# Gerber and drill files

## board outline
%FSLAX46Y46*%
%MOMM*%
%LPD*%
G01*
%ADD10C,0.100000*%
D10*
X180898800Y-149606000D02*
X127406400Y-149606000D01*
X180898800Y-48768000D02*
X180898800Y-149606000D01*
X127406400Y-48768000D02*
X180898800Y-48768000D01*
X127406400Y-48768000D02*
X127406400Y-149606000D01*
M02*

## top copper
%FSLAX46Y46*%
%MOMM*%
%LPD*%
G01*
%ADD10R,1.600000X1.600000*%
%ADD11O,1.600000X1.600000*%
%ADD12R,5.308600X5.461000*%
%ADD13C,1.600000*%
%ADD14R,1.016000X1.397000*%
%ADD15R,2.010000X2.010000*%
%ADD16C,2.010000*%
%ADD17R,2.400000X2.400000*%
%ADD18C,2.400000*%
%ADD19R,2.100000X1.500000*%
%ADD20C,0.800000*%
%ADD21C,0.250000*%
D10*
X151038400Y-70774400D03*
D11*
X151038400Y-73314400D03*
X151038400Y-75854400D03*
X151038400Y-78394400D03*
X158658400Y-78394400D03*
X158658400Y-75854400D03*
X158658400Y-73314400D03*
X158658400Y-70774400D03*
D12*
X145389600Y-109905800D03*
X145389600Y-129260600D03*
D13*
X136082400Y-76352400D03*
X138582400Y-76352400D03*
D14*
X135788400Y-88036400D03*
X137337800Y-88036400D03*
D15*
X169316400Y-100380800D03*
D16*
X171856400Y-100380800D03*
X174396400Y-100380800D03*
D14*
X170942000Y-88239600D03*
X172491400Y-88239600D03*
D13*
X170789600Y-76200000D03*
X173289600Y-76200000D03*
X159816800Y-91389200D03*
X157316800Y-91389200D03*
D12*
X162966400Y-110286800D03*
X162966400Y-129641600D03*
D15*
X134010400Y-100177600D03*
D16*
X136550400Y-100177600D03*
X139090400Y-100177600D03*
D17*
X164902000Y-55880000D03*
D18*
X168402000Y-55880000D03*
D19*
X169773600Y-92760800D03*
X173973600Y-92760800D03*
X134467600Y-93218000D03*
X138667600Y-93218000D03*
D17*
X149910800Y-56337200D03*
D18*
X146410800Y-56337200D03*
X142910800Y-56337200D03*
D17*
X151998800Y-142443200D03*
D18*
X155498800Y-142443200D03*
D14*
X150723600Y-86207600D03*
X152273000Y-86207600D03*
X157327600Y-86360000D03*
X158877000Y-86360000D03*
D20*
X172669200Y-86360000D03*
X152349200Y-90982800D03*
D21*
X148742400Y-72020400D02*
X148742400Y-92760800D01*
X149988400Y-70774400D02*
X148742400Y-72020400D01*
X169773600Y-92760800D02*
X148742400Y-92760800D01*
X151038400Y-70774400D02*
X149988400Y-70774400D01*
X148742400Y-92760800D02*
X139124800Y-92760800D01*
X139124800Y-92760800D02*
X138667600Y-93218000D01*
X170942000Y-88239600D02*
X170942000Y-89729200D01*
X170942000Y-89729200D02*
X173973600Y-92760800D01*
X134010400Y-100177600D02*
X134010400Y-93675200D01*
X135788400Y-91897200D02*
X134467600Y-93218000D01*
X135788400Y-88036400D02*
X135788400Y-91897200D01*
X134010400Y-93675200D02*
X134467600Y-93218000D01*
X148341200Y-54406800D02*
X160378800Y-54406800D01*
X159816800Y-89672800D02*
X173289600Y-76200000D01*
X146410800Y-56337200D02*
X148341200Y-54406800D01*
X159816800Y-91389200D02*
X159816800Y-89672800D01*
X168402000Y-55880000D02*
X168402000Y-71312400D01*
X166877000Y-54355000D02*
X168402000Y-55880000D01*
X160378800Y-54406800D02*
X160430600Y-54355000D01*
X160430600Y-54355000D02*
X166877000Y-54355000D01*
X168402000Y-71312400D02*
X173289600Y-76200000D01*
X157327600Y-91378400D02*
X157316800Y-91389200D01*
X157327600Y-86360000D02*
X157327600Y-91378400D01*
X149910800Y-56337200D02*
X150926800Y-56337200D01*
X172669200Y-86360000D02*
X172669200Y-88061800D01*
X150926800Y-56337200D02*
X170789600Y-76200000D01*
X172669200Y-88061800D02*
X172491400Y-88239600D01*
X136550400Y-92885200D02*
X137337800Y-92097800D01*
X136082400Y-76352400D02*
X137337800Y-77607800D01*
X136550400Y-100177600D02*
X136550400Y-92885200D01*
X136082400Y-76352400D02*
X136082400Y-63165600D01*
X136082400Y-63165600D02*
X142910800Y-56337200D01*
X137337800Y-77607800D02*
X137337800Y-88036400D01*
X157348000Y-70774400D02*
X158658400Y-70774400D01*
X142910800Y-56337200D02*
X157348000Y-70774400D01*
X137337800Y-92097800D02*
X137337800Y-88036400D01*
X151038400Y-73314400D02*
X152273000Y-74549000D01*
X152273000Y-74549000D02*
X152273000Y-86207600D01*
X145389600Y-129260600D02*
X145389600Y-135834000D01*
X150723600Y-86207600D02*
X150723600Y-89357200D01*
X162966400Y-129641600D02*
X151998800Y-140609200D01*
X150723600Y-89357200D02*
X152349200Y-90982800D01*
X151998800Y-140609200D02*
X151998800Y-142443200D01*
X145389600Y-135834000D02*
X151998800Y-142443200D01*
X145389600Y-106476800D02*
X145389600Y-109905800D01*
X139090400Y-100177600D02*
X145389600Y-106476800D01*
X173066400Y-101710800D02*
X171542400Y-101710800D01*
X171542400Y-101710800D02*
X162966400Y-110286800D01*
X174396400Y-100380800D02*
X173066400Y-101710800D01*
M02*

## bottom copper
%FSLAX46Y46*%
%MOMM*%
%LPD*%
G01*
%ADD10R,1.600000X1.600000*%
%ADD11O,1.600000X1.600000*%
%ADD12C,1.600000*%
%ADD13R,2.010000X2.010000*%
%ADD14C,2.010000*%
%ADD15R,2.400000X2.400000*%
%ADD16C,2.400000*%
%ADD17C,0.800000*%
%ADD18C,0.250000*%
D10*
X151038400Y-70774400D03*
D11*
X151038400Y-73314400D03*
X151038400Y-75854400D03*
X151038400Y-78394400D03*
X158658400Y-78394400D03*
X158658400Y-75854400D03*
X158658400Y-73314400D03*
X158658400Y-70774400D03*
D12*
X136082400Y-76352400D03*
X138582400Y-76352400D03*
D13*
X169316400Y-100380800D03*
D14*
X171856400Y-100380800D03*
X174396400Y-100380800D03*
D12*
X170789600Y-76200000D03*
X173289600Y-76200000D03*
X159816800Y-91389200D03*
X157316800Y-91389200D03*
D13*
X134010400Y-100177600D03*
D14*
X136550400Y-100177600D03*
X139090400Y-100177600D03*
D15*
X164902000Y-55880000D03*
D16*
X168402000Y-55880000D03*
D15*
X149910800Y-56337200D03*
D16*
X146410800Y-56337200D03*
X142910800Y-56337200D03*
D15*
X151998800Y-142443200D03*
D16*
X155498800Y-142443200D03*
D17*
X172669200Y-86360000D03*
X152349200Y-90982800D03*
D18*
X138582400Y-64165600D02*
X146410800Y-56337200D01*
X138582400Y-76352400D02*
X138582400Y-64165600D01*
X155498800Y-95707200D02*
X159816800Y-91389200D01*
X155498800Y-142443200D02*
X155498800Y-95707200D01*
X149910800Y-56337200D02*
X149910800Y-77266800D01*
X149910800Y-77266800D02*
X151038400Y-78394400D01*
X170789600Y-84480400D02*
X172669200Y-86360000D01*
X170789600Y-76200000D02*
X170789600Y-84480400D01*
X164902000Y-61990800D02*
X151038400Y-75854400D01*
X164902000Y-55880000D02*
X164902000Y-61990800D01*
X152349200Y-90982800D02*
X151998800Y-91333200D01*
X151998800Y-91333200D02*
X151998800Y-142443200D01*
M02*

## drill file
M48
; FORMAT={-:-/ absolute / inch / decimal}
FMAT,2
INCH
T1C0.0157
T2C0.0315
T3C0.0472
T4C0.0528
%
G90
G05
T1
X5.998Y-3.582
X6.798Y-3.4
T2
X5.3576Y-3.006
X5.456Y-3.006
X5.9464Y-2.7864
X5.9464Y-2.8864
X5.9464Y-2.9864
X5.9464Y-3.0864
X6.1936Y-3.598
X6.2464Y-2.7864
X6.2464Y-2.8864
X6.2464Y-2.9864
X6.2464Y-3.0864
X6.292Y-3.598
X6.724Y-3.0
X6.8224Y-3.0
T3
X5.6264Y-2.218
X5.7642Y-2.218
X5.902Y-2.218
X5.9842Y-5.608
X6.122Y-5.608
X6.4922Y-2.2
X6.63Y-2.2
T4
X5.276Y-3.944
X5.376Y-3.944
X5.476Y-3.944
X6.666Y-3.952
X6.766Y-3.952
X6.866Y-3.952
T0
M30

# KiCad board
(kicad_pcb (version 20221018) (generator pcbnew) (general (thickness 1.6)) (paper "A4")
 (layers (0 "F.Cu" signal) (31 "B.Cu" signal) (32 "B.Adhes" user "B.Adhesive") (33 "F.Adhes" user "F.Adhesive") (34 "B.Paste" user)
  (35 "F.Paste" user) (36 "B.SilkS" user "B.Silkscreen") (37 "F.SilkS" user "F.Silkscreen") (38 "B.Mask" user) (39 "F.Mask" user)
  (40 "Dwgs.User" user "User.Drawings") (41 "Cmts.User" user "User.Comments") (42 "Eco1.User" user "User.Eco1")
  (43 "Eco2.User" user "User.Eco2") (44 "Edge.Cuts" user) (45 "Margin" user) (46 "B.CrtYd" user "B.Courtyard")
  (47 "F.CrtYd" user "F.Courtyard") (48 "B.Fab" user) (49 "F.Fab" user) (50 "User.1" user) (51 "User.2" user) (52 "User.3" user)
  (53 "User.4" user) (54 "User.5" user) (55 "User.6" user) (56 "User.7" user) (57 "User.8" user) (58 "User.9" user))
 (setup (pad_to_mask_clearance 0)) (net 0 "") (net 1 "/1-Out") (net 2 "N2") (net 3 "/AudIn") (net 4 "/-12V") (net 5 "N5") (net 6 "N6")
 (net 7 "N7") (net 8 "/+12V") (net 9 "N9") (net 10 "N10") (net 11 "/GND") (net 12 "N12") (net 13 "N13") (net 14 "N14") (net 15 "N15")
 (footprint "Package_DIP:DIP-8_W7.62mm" (layer "F.Cu") (at 151.0384 70.7744)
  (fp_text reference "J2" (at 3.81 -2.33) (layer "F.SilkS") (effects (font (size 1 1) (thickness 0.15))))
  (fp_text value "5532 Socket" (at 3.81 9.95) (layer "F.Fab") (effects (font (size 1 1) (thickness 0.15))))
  (pad "1" thru_hole rect (at 0 0) (size 1.6 1.6) (drill 0.8) (layers "*.Cu" "*.Mask") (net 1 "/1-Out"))
  (pad "2" thru_hole oval (at 0 2.54) (size 1.6 1.6) (drill 0.8) (layers "*.Cu" "*.Mask") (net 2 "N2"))
  (pad "3" thru_hole oval (at 0 5.08) (size 1.6 1.6) (drill 0.8) (layers "*.Cu" "*.Mask") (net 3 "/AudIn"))
  (pad "4" thru_hole oval (at 0 7.62) (size 1.6 1.6) (drill 0.8) (layers "*.Cu" "*.Mask") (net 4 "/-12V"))
  (pad "5" thru_hole oval (at 7.62 7.62) (size 1.6 1.6) (drill 0.8) (layers "*.Cu" "*.Mask") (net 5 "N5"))
  (pad "6" thru_hole oval (at 7.62 5.08) (size 1.6 1.6) (drill 0.8) (layers "*.Cu" "*.Mask") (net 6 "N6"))
  (pad "7" thru_hole oval (at 7.62 2.54) (size 1.6 1.6) (drill 0.8) (layers "*.Cu" "*.Mask") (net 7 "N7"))
  (pad "8" thru_hole oval (at 7.62 0) (size 1.6 1.6) (drill 0.8) (layers "*.Cu" "*.Mask") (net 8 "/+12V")))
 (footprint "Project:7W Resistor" (layer "F.Cu") (at 145.3896 119.5832 -90)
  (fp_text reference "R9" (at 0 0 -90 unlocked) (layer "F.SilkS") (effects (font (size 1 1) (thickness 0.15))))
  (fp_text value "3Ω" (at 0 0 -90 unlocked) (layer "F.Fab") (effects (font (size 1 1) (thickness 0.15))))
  (pad "1" smd rect (at -9.6774 0) (size 5.3086 5.461) (layers "F.Cu" "F.Paste" "F.Mask") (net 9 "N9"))
  (pad "2" smd rect (at 9.6774 0) (size 5.3086 5.461) (layers "F.Cu" "F.Paste" "F.Mask") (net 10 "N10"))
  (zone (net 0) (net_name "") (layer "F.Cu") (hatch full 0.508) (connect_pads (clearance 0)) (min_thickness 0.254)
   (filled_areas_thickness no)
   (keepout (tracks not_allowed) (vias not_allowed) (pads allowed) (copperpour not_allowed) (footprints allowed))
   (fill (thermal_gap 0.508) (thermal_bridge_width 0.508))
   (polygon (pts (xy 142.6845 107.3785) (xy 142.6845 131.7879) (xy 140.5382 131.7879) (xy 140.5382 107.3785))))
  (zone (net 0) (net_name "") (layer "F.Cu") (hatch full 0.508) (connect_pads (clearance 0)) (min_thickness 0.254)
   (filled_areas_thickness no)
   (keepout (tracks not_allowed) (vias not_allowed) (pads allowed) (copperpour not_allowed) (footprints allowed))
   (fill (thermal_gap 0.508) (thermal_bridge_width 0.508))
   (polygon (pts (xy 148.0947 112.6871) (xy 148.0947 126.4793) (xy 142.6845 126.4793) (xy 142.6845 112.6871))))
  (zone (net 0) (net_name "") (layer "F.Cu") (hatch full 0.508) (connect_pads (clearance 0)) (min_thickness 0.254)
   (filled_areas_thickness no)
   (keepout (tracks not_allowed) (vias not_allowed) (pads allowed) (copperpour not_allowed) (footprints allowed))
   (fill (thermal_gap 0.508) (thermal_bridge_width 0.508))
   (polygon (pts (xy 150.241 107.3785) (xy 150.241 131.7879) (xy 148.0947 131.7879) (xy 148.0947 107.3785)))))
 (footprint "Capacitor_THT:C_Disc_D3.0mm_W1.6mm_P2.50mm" (layer "F.Cu") (at 136.0824 76.3524)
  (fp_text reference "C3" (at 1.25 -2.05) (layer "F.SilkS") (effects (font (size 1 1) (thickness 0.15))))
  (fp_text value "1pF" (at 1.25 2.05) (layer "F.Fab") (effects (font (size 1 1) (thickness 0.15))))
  (pad "1" thru_hole circle (at 0 0) (size 1.6 1.6) (drill 0.8) (layers "*.Cu" "*.Mask") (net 8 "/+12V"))
  (pad "2" thru_hole circle (at 2.5 0) (size 1.6 1.6) (drill 0.8) (layers "*.Cu" "*.Mask") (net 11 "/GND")))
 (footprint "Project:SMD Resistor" (layer "F.Cu") (at 136.5631 88.0364)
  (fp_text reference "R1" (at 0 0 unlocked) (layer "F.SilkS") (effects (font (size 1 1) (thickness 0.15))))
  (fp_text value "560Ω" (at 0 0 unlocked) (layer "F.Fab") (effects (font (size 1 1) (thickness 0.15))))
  (pad "1" smd rect (at -0.7747 0) (size 1.016 1.397) (layers "F.Cu" "F.Paste" "F.Mask") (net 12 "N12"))
  (pad "2" smd rect (at 0.7747 0) (size 1.016 1.397) (layers "F.Cu" "F.Paste" "F.Mask") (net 8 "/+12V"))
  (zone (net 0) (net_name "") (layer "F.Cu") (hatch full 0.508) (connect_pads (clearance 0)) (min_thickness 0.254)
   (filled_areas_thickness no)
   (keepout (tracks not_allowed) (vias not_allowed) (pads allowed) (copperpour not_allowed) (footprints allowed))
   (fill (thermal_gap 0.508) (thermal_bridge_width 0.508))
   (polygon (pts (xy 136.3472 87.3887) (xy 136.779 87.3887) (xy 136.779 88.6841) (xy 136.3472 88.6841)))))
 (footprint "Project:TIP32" (layer "F.Cu") (at 169.3164 100.3808)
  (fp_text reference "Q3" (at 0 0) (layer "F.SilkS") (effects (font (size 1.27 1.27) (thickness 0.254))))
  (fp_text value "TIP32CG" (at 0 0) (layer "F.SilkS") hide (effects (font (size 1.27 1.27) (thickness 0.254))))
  (pad "1" thru_hole rect (at 0 0) (size 2.01 2.01) (drill 1.34) (layers "*.Cu" "*.Mask") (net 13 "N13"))
  (pad "2" thru_hole circle (at 2.54 0) (size 2.01 2.01) (drill 1.34) (layers "*.Cu" "*.Mask") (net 4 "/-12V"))
  (pad "3" thru_hole circle (at 5.08 0) (size 2.01 2.01) (drill 1.34) (layers "*.Cu" "*.Mask") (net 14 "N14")))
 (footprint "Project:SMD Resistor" (layer "F.Cu") (at 171.7167 88.2396)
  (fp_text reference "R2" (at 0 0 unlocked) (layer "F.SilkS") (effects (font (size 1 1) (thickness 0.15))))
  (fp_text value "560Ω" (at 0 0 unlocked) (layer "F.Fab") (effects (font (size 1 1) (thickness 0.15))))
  (pad "1" smd rect (at -0.7747 0) (size 1.016 1.397) (layers "F.Cu" "F.Paste" "F.Mask") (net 13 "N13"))
  (pad "2" smd rect (at 0.7747 0) (size 1.016 1.397) (layers "F.Cu" "F.Paste" "F.Mask") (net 4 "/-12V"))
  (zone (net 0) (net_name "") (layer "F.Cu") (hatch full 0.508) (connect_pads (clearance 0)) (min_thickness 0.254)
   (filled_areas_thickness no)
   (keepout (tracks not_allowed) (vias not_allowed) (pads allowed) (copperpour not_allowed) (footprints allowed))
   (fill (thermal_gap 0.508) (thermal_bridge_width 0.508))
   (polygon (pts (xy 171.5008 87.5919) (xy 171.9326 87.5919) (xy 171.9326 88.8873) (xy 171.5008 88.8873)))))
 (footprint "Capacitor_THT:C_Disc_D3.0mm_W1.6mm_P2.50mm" (layer "F.Cu") (at 170.7896 76.2)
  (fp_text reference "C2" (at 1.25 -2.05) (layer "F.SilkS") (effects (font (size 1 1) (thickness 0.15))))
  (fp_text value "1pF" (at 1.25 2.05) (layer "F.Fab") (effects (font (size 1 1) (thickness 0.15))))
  (pad "1" thru_hole circle (at 0 0) (size 1.6 1.6) (drill 0.8) (layers "*.Cu" "*.Mask") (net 4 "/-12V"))
  (pad "2" thru_hole circle (at 2.5 0) (size 1.6 1.6) (drill 0.8) (layers "*.Cu" "*.Mask") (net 11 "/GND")))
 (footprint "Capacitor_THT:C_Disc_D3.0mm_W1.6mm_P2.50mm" (layer "F.Cu") (at 159.8168 91.3892 180)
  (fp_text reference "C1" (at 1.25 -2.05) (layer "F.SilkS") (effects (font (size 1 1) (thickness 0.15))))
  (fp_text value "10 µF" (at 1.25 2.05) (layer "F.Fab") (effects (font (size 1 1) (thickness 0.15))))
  (pad "1" thru_hole circle (at 0 0 180) (size 1.6 1.6) (drill 0.8) (layers "*.Cu" "*.Mask") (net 11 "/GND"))
  (pad "2" thru_hole circle (at 2.5 0 180) (size 1.6 1.6) (drill 0.8) (layers "*.Cu" "*.Mask") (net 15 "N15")))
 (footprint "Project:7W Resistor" (layer "F.Cu") (at 162.9664 119.9642 -90)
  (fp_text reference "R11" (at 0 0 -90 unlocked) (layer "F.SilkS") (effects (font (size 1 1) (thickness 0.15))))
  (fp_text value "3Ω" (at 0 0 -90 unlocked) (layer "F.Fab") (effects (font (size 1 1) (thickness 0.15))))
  (pad "1" smd rect (at -9.6774 0) (size 5.3086 5.461) (layers "F.Cu" "F.Paste" "F.Mask") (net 14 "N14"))
  (pad "2" smd rect (at 9.6774 0) (size 5.3086 5.461) (layers "F.Cu" "F.Paste" "F.Mask") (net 10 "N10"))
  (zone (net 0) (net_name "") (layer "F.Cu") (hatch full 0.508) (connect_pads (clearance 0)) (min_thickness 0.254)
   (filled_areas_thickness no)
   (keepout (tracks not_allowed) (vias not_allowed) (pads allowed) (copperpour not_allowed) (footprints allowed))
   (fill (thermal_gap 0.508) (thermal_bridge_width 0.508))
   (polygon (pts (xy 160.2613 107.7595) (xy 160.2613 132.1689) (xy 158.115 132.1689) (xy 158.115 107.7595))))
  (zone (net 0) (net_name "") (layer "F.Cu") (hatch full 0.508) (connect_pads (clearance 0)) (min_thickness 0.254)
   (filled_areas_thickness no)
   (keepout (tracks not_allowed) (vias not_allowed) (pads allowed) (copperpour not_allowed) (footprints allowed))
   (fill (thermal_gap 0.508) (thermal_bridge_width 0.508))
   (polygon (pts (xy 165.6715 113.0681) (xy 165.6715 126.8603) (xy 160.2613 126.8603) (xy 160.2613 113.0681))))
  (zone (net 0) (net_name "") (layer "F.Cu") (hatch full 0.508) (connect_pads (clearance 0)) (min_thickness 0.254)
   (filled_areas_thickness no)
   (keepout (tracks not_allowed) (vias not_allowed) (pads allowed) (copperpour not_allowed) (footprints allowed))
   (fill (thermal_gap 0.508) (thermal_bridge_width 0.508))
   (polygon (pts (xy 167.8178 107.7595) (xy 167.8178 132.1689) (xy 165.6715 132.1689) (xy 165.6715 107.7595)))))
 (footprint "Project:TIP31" (layer "F.Cu") (at 134.0104 100.1776)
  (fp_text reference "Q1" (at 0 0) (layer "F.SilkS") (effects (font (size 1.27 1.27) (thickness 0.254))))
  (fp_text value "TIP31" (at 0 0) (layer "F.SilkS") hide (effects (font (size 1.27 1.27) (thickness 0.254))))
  (pad "1" thru_hole rect (at 0 0) (size 2.01 2.01) (drill 1.34) (layers "*.Cu" "*.Mask") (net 12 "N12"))
  (pad "2" thru_hole circle (at 2.54 0) (size 2.01 2.01) (drill 1.34) (layers "*.Cu" "*.Mask") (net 8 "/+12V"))
  (pad "3" thru_hole circle (at 5.08 0) (size 2.01 2.01) (drill 1.34) (layers "*.Cu" "*.Mask") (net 9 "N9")))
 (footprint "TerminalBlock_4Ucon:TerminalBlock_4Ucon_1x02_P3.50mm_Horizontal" (layer "F.Cu") (at 164.902 55.88)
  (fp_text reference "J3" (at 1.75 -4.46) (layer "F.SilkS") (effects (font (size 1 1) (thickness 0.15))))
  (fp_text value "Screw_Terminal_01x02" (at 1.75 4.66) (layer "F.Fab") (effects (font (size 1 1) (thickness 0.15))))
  (pad "1" thru_hole rect (at 0 0) (size 2.4 2.4) (drill 1.2) (layers "*.Cu" "*.Mask") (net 3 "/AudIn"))
  (pad "2" thru_hole circle (at 3.5 0) (size 2.4 2.4) (drill 1.2) (layers "*.Cu" "*.Mask") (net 11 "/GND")))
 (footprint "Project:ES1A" (layer "F.Cu") (at 171.8736 92.7608)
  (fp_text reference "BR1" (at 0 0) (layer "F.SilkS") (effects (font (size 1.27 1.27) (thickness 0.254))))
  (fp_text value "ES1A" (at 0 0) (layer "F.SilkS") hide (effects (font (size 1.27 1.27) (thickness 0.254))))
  (pad "1" smd rect (at -2.1 0 90) (size 1.5 2.1) (layers "F.Cu" "F.Paste" "F.Mask") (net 1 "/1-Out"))
  (pad "2" smd rect (at 2.1 0 90) (size 1.5 2.1) (layers "F.Cu" "F.Paste" "F.Mask") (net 13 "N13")))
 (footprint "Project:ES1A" (layer "F.Cu") (at 136.5676 93.218)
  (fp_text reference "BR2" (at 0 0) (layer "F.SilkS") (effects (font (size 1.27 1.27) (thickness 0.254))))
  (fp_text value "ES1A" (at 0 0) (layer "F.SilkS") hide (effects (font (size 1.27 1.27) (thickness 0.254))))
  (pad "1" smd rect (at -2.1 0 90) (size 1.5 2.1) (layers "F.Cu" "F.Paste" "F.Mask") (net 12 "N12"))
  (pad "2" smd rect (at 2.1 0 90) (size 1.5 2.1) (layers "F.Cu" "F.Paste" "F.Mask") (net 1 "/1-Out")))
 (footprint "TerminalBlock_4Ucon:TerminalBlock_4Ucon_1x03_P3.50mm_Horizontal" (layer "F.Cu") (at 149.9108 56.3372 180)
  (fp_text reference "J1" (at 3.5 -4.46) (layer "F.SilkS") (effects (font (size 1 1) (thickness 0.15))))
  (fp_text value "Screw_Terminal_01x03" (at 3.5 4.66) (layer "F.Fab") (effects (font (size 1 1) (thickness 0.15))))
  (pad "1" thru_hole rect (at 0 0 180) (size 2.4 2.4) (drill 1.2) (layers "*.Cu" "*.Mask") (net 4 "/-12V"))
  (pad "2" thru_hole circle (at 3.5 0 180) (size 2.4 2.4) (drill 1.2) (layers "*.Cu" "*.Mask") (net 11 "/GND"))
  (pad "3" thru_hole circle (at 7 0 180) (size 2.4 2.4) (drill 1.2) (layers "*.Cu" "*.Mask") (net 8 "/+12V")))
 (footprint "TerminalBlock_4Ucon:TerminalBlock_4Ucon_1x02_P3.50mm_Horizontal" (layer "F.Cu") (at 151.9988 142.4432)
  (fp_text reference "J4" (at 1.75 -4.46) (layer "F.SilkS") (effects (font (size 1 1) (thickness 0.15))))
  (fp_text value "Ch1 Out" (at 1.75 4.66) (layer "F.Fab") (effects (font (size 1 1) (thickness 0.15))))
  (pad "1" thru_hole rect (at 0 0) (size 2.4 2.4) (drill 1.2) (layers "*.Cu" "*.Mask") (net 10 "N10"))
  (pad "2" thru_hole circle (at 3.5 0) (size 2.4 2.4) (drill 1.2) (layers "*.Cu" "*.Mask") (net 11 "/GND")))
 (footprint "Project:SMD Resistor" (layer "F.Cu") (at 151.4983 86.2076)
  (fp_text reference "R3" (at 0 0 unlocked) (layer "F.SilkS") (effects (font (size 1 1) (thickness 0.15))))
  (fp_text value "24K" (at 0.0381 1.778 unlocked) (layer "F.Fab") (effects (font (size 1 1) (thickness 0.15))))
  (pad "1" smd rect (at -0.7747 0) (size 1.016 1.397) (layers "F.Cu" "F.Paste" "F.Mask") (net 10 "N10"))
  (pad "2" smd rect (at 0.7747 0) (size 1.016 1.397) (layers "F.Cu" "F.Paste" "F.Mask") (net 2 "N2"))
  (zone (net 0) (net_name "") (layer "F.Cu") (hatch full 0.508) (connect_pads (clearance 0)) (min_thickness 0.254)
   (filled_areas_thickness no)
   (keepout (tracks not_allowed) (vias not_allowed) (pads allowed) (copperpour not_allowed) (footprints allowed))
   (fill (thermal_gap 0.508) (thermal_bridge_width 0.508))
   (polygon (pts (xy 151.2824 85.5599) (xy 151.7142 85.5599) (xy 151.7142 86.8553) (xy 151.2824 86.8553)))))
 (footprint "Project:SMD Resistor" (layer "F.Cu") (at 158.1023 86.36)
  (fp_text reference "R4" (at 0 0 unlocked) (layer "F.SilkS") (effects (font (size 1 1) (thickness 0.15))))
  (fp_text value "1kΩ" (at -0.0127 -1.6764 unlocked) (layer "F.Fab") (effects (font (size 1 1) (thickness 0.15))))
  (pad "1" smd rect (at -0.7747 0) (size 1.016 1.397) (layers "F.Cu" "F.Paste" "F.Mask") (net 15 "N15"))
  (pad "2" smd rect (at 0.7747 0) (size 1.016 1.397) (layers "F.Cu" "F.Paste" "F.Mask") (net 2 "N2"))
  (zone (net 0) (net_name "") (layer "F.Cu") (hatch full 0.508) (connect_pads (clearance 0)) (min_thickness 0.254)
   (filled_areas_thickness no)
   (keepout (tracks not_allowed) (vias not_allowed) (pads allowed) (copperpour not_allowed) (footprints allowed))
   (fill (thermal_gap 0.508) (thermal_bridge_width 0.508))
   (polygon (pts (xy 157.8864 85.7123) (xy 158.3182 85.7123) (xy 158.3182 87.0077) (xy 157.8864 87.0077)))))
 (gr_line (start 180.8988 149.606) (end 127.4064 149.606) (stroke (width 0.1) (type default)) (layer "Edge.Cuts"))
 (gr_line (start 180.8988 48.768) (end 180.8988 149.606) (stroke (width 0.1) (type default)) (layer "Edge.Cuts"))
 (gr_line (start 127.4064 48.768) (end 180.8988 48.768) (stroke (width 0.1) (type default)) (layer "Edge.Cuts"))
 (gr_line (start 127.4064 48.768) (end 127.4064 149.606) (stroke (width 0.1) (type default)) (layer "Edge.Cuts"))
 (segment (start 148.7424 72.0204) (end 148.7424 92.7608) (width 0.25) (layer "F.Cu") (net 1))
 (segment (start 149.9884 70.7744) (end 148.7424 72.0204) (width 0.25) (layer "F.Cu") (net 1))
 (segment (start 169.7736 92.7608) (end 148.7424 92.7608) (width 0.25) (layer "F.Cu") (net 1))
 (segment (start 151.0384 70.7744) (end 149.9884 70.7744) (width 0.25) (layer "F.Cu") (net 1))
 (segment (start 148.7424 92.7608) (end 139.1248 92.7608) (width 0.25) (layer "F.Cu") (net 1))
 (segment (start 139.1248 92.7608) (end 138.6676 93.218) (width 0.25) (layer "F.Cu") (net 1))
 (segment (start 170.942 88.2396) (end 170.942 89.7292) (width 0.25) (layer "F.Cu") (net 13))
 (segment (start 170.942 89.7292) (end 173.9736 92.7608) (width 0.25) (layer "F.Cu") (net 13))
 (segment (start 134.0104 100.1776) (end 134.0104 93.6752) (width 0.25) (layer "F.Cu") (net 12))
 (segment (start 135.7884 91.8972) (end 134.4676 93.218) (width 0.25) (layer "F.Cu") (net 12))
 (segment (start 135.7884 88.0364) (end 135.7884 91.8972) (width 0.25) (layer "F.Cu") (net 12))
 (segment (start 134.0104 93.6752) (end 134.4676 93.218) (width 0.25) (layer "F.Cu") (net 12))
 (segment (start 148.3412 54.4068) (end 160.3788 54.4068) (width 0.25) (layer "F.Cu") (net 11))
 (segment (start 159.8168 89.6728) (end 173.2896 76.2) (width 0.25) (layer "F.Cu") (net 11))
 (segment (start 146.4108 56.3372) (end 148.3412 54.4068) (width 0.25) (layer "F.Cu") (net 11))
 (segment (start 159.8168 91.3892) (end 159.8168 89.6728) (width 0.25) (layer "F.Cu") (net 11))
 (segment (start 168.402 55.88) (end 168.402 71.3124) (width 0.25) (layer "F.Cu") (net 11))
 (segment (start 166.877 54.355) (end 168.402 55.88) (width 0.25) (layer "F.Cu") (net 11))
 (segment (start 160.3788 54.4068) (end 160.4306 54.355) (width 0.25) (layer "F.Cu") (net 11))
 (segment (start 160.4306 54.355) (end 166.877 54.355) (width 0.25) (layer "F.Cu") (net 11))
 (segment (start 168.402 71.3124) (end 173.2896 76.2) (width 0.25) (layer "F.Cu") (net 11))
 (segment (start 138.5824 64.1656) (end 146.4108 56.3372) (width 0.25) (layer "B.Cu") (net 11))
 (segment (start 138.5824 76.3524) (end 138.5824 64.1656) (width 0.25) (layer "B.Cu") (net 11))
 (segment (start 155.4988 95.7072) (end 159.8168 91.3892) (width 0.25) (layer "B.Cu") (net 11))
 (segment (start 155.4988 142.4432) (end 155.4988 95.7072) (width 0.25) (layer "B.Cu") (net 11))
 (segment (start 157.3276 91.3784) (end 157.3168 91.3892) (width 0.25) (layer "F.Cu") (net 15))
 (segment (start 157.3276 86.36) (end 157.3276 91.3784) (width 0.25) (layer "F.Cu") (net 15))
 (segment (start 149.9108 56.3372) (end 150.9268 56.3372) (width 0.25) (layer "F.Cu") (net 4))
 (segment (start 172.6692 86.36) (end 172.6692 88.0618) (width 0.25) (layer "F.Cu") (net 4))
 (segment (start 150.9268 56.3372) (end 170.7896 76.2) (width 0.25) (layer "F.Cu") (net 4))
 (segment (start 172.6692 88.0618) (end 172.4914 88.2396) (width 0.25) (layer "F.Cu") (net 4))
 (via (at 172.6692 86.36) (size 0.8) (drill 0.4) (layers "F.Cu" "B.Cu") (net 4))
 (segment (start 149.9108 56.3372) (end 149.9108 77.2668) (width 0.25) (layer "B.Cu") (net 4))
 (segment (start 149.9108 77.2668) (end 151.0384 78.3944) (width 0.25) (layer "B.Cu") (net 4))
 (segment (start 170.7896 84.4804) (end 172.6692 86.36) (width 0.25) (layer "B.Cu") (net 4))
 (segment (start 170.7896 76.2) (end 170.7896 84.4804) (width 0.25) (layer "B.Cu") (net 4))
 (segment (start 136.5504 92.8852) (end 137.3378 92.0978) (width 0.25) (layer "F.Cu") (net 8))
 (segment (start 136.0824 76.3524) (end 137.3378 77.6078) (width 0.25) (layer "F.Cu") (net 8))
 (segment (start 136.5504 100.1776) (end 136.5504 92.8852) (width 0.25) (layer "F.Cu") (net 8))
 (segment (start 136.0824 76.3524) (end 136.0824 63.1656) (width 0.25) (layer "F.Cu") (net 8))
 (segment (start 136.0824 63.1656) (end 142.9108 56.3372) (width 0.25) (layer "F.Cu") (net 8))
 (segment (start 137.3378 77.6078) (end 137.3378 88.0364) (width 0.25) (layer "F.Cu") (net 8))
 (segment (start 157.348 70.7744) (end 158.6584 70.7744) (width 0.25) (layer "F.Cu") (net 8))
 (segment (start 142.9108 56.3372) (end 157.348 70.7744) (width 0.25) (layer "F.Cu") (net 8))
 (segment (start 137.3378 92.0978) (end 137.3378 88.0364) (width 0.25) (layer "F.Cu") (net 8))
 (segment (start 151.0384 73.3144) (end 152.273 74.549) (width 0.25) (layer "F.Cu") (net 2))
 (segment (start 152.273 74.549) (end 152.273 86.2076) (width 0.25) (layer "F.Cu") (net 2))
 (segment (start 164.902 61.9908) (end 151.0384 75.8544) (width 0.25) (layer "B.Cu") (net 3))
 (segment (start 164.902 55.88) (end 164.902 61.9908) (width 0.25) (layer "B.Cu") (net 3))
 (segment (start 145.3896 129.2606) (end 145.3896 135.834) (width 0.25) (layer "F.Cu") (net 10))
 (segment (start 150.7236 86.2076) (end 150.7236 89.3572) (width 0.25) (layer "F.Cu") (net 10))
 (segment (start 162.9664 129.6416) (end 151.9988 140.6092) (width 0.25) (layer "F.Cu") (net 10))
 (segment (start 150.7236 89.3572) (end 152.3492 90.9828) (width 0.25) (layer "F.Cu") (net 10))
 (segment (start 151.9988 140.6092) (end 151.9988 142.4432) (width 0.25) (layer "F.Cu") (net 10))
 (segment (start 145.3896 135.834) (end 151.9988 142.4432) (width 0.25) (layer "F.Cu") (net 10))
 (via (at 152.3492 90.9828) (size 0.8) (drill 0.4) (layers "F.Cu" "B.Cu") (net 10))
 (segment (start 152.3492 90.9828) (end 151.9988 91.3332) (width 0.25) (layer "B.Cu") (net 10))
 (segment (start 151.9988 91.3332) (end 151.9988 142.4432) (width 0.25) (layer "B.Cu") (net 10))
 (segment (start 145.3896 106.4768) (end 145.3896 109.9058) (width 0.25) (layer "F.Cu") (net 9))
 (segment (start 139.0904 100.1776) (end 145.3896 106.4768) (width 0.25) (layer "F.Cu") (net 9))
 (segment (start 173.0664 101.7108) (end 171.5424 101.7108) (width 0.25) (layer "F.Cu") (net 14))
 (segment (start 171.5424 101.7108) (end 162.9664 110.2868) (width 0.25) (layer "F.Cu") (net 14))
 (segment (start 174.3964 100.3808) (end 173.0664 101.7108) (width 0.25) (layer "F.Cu") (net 14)))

